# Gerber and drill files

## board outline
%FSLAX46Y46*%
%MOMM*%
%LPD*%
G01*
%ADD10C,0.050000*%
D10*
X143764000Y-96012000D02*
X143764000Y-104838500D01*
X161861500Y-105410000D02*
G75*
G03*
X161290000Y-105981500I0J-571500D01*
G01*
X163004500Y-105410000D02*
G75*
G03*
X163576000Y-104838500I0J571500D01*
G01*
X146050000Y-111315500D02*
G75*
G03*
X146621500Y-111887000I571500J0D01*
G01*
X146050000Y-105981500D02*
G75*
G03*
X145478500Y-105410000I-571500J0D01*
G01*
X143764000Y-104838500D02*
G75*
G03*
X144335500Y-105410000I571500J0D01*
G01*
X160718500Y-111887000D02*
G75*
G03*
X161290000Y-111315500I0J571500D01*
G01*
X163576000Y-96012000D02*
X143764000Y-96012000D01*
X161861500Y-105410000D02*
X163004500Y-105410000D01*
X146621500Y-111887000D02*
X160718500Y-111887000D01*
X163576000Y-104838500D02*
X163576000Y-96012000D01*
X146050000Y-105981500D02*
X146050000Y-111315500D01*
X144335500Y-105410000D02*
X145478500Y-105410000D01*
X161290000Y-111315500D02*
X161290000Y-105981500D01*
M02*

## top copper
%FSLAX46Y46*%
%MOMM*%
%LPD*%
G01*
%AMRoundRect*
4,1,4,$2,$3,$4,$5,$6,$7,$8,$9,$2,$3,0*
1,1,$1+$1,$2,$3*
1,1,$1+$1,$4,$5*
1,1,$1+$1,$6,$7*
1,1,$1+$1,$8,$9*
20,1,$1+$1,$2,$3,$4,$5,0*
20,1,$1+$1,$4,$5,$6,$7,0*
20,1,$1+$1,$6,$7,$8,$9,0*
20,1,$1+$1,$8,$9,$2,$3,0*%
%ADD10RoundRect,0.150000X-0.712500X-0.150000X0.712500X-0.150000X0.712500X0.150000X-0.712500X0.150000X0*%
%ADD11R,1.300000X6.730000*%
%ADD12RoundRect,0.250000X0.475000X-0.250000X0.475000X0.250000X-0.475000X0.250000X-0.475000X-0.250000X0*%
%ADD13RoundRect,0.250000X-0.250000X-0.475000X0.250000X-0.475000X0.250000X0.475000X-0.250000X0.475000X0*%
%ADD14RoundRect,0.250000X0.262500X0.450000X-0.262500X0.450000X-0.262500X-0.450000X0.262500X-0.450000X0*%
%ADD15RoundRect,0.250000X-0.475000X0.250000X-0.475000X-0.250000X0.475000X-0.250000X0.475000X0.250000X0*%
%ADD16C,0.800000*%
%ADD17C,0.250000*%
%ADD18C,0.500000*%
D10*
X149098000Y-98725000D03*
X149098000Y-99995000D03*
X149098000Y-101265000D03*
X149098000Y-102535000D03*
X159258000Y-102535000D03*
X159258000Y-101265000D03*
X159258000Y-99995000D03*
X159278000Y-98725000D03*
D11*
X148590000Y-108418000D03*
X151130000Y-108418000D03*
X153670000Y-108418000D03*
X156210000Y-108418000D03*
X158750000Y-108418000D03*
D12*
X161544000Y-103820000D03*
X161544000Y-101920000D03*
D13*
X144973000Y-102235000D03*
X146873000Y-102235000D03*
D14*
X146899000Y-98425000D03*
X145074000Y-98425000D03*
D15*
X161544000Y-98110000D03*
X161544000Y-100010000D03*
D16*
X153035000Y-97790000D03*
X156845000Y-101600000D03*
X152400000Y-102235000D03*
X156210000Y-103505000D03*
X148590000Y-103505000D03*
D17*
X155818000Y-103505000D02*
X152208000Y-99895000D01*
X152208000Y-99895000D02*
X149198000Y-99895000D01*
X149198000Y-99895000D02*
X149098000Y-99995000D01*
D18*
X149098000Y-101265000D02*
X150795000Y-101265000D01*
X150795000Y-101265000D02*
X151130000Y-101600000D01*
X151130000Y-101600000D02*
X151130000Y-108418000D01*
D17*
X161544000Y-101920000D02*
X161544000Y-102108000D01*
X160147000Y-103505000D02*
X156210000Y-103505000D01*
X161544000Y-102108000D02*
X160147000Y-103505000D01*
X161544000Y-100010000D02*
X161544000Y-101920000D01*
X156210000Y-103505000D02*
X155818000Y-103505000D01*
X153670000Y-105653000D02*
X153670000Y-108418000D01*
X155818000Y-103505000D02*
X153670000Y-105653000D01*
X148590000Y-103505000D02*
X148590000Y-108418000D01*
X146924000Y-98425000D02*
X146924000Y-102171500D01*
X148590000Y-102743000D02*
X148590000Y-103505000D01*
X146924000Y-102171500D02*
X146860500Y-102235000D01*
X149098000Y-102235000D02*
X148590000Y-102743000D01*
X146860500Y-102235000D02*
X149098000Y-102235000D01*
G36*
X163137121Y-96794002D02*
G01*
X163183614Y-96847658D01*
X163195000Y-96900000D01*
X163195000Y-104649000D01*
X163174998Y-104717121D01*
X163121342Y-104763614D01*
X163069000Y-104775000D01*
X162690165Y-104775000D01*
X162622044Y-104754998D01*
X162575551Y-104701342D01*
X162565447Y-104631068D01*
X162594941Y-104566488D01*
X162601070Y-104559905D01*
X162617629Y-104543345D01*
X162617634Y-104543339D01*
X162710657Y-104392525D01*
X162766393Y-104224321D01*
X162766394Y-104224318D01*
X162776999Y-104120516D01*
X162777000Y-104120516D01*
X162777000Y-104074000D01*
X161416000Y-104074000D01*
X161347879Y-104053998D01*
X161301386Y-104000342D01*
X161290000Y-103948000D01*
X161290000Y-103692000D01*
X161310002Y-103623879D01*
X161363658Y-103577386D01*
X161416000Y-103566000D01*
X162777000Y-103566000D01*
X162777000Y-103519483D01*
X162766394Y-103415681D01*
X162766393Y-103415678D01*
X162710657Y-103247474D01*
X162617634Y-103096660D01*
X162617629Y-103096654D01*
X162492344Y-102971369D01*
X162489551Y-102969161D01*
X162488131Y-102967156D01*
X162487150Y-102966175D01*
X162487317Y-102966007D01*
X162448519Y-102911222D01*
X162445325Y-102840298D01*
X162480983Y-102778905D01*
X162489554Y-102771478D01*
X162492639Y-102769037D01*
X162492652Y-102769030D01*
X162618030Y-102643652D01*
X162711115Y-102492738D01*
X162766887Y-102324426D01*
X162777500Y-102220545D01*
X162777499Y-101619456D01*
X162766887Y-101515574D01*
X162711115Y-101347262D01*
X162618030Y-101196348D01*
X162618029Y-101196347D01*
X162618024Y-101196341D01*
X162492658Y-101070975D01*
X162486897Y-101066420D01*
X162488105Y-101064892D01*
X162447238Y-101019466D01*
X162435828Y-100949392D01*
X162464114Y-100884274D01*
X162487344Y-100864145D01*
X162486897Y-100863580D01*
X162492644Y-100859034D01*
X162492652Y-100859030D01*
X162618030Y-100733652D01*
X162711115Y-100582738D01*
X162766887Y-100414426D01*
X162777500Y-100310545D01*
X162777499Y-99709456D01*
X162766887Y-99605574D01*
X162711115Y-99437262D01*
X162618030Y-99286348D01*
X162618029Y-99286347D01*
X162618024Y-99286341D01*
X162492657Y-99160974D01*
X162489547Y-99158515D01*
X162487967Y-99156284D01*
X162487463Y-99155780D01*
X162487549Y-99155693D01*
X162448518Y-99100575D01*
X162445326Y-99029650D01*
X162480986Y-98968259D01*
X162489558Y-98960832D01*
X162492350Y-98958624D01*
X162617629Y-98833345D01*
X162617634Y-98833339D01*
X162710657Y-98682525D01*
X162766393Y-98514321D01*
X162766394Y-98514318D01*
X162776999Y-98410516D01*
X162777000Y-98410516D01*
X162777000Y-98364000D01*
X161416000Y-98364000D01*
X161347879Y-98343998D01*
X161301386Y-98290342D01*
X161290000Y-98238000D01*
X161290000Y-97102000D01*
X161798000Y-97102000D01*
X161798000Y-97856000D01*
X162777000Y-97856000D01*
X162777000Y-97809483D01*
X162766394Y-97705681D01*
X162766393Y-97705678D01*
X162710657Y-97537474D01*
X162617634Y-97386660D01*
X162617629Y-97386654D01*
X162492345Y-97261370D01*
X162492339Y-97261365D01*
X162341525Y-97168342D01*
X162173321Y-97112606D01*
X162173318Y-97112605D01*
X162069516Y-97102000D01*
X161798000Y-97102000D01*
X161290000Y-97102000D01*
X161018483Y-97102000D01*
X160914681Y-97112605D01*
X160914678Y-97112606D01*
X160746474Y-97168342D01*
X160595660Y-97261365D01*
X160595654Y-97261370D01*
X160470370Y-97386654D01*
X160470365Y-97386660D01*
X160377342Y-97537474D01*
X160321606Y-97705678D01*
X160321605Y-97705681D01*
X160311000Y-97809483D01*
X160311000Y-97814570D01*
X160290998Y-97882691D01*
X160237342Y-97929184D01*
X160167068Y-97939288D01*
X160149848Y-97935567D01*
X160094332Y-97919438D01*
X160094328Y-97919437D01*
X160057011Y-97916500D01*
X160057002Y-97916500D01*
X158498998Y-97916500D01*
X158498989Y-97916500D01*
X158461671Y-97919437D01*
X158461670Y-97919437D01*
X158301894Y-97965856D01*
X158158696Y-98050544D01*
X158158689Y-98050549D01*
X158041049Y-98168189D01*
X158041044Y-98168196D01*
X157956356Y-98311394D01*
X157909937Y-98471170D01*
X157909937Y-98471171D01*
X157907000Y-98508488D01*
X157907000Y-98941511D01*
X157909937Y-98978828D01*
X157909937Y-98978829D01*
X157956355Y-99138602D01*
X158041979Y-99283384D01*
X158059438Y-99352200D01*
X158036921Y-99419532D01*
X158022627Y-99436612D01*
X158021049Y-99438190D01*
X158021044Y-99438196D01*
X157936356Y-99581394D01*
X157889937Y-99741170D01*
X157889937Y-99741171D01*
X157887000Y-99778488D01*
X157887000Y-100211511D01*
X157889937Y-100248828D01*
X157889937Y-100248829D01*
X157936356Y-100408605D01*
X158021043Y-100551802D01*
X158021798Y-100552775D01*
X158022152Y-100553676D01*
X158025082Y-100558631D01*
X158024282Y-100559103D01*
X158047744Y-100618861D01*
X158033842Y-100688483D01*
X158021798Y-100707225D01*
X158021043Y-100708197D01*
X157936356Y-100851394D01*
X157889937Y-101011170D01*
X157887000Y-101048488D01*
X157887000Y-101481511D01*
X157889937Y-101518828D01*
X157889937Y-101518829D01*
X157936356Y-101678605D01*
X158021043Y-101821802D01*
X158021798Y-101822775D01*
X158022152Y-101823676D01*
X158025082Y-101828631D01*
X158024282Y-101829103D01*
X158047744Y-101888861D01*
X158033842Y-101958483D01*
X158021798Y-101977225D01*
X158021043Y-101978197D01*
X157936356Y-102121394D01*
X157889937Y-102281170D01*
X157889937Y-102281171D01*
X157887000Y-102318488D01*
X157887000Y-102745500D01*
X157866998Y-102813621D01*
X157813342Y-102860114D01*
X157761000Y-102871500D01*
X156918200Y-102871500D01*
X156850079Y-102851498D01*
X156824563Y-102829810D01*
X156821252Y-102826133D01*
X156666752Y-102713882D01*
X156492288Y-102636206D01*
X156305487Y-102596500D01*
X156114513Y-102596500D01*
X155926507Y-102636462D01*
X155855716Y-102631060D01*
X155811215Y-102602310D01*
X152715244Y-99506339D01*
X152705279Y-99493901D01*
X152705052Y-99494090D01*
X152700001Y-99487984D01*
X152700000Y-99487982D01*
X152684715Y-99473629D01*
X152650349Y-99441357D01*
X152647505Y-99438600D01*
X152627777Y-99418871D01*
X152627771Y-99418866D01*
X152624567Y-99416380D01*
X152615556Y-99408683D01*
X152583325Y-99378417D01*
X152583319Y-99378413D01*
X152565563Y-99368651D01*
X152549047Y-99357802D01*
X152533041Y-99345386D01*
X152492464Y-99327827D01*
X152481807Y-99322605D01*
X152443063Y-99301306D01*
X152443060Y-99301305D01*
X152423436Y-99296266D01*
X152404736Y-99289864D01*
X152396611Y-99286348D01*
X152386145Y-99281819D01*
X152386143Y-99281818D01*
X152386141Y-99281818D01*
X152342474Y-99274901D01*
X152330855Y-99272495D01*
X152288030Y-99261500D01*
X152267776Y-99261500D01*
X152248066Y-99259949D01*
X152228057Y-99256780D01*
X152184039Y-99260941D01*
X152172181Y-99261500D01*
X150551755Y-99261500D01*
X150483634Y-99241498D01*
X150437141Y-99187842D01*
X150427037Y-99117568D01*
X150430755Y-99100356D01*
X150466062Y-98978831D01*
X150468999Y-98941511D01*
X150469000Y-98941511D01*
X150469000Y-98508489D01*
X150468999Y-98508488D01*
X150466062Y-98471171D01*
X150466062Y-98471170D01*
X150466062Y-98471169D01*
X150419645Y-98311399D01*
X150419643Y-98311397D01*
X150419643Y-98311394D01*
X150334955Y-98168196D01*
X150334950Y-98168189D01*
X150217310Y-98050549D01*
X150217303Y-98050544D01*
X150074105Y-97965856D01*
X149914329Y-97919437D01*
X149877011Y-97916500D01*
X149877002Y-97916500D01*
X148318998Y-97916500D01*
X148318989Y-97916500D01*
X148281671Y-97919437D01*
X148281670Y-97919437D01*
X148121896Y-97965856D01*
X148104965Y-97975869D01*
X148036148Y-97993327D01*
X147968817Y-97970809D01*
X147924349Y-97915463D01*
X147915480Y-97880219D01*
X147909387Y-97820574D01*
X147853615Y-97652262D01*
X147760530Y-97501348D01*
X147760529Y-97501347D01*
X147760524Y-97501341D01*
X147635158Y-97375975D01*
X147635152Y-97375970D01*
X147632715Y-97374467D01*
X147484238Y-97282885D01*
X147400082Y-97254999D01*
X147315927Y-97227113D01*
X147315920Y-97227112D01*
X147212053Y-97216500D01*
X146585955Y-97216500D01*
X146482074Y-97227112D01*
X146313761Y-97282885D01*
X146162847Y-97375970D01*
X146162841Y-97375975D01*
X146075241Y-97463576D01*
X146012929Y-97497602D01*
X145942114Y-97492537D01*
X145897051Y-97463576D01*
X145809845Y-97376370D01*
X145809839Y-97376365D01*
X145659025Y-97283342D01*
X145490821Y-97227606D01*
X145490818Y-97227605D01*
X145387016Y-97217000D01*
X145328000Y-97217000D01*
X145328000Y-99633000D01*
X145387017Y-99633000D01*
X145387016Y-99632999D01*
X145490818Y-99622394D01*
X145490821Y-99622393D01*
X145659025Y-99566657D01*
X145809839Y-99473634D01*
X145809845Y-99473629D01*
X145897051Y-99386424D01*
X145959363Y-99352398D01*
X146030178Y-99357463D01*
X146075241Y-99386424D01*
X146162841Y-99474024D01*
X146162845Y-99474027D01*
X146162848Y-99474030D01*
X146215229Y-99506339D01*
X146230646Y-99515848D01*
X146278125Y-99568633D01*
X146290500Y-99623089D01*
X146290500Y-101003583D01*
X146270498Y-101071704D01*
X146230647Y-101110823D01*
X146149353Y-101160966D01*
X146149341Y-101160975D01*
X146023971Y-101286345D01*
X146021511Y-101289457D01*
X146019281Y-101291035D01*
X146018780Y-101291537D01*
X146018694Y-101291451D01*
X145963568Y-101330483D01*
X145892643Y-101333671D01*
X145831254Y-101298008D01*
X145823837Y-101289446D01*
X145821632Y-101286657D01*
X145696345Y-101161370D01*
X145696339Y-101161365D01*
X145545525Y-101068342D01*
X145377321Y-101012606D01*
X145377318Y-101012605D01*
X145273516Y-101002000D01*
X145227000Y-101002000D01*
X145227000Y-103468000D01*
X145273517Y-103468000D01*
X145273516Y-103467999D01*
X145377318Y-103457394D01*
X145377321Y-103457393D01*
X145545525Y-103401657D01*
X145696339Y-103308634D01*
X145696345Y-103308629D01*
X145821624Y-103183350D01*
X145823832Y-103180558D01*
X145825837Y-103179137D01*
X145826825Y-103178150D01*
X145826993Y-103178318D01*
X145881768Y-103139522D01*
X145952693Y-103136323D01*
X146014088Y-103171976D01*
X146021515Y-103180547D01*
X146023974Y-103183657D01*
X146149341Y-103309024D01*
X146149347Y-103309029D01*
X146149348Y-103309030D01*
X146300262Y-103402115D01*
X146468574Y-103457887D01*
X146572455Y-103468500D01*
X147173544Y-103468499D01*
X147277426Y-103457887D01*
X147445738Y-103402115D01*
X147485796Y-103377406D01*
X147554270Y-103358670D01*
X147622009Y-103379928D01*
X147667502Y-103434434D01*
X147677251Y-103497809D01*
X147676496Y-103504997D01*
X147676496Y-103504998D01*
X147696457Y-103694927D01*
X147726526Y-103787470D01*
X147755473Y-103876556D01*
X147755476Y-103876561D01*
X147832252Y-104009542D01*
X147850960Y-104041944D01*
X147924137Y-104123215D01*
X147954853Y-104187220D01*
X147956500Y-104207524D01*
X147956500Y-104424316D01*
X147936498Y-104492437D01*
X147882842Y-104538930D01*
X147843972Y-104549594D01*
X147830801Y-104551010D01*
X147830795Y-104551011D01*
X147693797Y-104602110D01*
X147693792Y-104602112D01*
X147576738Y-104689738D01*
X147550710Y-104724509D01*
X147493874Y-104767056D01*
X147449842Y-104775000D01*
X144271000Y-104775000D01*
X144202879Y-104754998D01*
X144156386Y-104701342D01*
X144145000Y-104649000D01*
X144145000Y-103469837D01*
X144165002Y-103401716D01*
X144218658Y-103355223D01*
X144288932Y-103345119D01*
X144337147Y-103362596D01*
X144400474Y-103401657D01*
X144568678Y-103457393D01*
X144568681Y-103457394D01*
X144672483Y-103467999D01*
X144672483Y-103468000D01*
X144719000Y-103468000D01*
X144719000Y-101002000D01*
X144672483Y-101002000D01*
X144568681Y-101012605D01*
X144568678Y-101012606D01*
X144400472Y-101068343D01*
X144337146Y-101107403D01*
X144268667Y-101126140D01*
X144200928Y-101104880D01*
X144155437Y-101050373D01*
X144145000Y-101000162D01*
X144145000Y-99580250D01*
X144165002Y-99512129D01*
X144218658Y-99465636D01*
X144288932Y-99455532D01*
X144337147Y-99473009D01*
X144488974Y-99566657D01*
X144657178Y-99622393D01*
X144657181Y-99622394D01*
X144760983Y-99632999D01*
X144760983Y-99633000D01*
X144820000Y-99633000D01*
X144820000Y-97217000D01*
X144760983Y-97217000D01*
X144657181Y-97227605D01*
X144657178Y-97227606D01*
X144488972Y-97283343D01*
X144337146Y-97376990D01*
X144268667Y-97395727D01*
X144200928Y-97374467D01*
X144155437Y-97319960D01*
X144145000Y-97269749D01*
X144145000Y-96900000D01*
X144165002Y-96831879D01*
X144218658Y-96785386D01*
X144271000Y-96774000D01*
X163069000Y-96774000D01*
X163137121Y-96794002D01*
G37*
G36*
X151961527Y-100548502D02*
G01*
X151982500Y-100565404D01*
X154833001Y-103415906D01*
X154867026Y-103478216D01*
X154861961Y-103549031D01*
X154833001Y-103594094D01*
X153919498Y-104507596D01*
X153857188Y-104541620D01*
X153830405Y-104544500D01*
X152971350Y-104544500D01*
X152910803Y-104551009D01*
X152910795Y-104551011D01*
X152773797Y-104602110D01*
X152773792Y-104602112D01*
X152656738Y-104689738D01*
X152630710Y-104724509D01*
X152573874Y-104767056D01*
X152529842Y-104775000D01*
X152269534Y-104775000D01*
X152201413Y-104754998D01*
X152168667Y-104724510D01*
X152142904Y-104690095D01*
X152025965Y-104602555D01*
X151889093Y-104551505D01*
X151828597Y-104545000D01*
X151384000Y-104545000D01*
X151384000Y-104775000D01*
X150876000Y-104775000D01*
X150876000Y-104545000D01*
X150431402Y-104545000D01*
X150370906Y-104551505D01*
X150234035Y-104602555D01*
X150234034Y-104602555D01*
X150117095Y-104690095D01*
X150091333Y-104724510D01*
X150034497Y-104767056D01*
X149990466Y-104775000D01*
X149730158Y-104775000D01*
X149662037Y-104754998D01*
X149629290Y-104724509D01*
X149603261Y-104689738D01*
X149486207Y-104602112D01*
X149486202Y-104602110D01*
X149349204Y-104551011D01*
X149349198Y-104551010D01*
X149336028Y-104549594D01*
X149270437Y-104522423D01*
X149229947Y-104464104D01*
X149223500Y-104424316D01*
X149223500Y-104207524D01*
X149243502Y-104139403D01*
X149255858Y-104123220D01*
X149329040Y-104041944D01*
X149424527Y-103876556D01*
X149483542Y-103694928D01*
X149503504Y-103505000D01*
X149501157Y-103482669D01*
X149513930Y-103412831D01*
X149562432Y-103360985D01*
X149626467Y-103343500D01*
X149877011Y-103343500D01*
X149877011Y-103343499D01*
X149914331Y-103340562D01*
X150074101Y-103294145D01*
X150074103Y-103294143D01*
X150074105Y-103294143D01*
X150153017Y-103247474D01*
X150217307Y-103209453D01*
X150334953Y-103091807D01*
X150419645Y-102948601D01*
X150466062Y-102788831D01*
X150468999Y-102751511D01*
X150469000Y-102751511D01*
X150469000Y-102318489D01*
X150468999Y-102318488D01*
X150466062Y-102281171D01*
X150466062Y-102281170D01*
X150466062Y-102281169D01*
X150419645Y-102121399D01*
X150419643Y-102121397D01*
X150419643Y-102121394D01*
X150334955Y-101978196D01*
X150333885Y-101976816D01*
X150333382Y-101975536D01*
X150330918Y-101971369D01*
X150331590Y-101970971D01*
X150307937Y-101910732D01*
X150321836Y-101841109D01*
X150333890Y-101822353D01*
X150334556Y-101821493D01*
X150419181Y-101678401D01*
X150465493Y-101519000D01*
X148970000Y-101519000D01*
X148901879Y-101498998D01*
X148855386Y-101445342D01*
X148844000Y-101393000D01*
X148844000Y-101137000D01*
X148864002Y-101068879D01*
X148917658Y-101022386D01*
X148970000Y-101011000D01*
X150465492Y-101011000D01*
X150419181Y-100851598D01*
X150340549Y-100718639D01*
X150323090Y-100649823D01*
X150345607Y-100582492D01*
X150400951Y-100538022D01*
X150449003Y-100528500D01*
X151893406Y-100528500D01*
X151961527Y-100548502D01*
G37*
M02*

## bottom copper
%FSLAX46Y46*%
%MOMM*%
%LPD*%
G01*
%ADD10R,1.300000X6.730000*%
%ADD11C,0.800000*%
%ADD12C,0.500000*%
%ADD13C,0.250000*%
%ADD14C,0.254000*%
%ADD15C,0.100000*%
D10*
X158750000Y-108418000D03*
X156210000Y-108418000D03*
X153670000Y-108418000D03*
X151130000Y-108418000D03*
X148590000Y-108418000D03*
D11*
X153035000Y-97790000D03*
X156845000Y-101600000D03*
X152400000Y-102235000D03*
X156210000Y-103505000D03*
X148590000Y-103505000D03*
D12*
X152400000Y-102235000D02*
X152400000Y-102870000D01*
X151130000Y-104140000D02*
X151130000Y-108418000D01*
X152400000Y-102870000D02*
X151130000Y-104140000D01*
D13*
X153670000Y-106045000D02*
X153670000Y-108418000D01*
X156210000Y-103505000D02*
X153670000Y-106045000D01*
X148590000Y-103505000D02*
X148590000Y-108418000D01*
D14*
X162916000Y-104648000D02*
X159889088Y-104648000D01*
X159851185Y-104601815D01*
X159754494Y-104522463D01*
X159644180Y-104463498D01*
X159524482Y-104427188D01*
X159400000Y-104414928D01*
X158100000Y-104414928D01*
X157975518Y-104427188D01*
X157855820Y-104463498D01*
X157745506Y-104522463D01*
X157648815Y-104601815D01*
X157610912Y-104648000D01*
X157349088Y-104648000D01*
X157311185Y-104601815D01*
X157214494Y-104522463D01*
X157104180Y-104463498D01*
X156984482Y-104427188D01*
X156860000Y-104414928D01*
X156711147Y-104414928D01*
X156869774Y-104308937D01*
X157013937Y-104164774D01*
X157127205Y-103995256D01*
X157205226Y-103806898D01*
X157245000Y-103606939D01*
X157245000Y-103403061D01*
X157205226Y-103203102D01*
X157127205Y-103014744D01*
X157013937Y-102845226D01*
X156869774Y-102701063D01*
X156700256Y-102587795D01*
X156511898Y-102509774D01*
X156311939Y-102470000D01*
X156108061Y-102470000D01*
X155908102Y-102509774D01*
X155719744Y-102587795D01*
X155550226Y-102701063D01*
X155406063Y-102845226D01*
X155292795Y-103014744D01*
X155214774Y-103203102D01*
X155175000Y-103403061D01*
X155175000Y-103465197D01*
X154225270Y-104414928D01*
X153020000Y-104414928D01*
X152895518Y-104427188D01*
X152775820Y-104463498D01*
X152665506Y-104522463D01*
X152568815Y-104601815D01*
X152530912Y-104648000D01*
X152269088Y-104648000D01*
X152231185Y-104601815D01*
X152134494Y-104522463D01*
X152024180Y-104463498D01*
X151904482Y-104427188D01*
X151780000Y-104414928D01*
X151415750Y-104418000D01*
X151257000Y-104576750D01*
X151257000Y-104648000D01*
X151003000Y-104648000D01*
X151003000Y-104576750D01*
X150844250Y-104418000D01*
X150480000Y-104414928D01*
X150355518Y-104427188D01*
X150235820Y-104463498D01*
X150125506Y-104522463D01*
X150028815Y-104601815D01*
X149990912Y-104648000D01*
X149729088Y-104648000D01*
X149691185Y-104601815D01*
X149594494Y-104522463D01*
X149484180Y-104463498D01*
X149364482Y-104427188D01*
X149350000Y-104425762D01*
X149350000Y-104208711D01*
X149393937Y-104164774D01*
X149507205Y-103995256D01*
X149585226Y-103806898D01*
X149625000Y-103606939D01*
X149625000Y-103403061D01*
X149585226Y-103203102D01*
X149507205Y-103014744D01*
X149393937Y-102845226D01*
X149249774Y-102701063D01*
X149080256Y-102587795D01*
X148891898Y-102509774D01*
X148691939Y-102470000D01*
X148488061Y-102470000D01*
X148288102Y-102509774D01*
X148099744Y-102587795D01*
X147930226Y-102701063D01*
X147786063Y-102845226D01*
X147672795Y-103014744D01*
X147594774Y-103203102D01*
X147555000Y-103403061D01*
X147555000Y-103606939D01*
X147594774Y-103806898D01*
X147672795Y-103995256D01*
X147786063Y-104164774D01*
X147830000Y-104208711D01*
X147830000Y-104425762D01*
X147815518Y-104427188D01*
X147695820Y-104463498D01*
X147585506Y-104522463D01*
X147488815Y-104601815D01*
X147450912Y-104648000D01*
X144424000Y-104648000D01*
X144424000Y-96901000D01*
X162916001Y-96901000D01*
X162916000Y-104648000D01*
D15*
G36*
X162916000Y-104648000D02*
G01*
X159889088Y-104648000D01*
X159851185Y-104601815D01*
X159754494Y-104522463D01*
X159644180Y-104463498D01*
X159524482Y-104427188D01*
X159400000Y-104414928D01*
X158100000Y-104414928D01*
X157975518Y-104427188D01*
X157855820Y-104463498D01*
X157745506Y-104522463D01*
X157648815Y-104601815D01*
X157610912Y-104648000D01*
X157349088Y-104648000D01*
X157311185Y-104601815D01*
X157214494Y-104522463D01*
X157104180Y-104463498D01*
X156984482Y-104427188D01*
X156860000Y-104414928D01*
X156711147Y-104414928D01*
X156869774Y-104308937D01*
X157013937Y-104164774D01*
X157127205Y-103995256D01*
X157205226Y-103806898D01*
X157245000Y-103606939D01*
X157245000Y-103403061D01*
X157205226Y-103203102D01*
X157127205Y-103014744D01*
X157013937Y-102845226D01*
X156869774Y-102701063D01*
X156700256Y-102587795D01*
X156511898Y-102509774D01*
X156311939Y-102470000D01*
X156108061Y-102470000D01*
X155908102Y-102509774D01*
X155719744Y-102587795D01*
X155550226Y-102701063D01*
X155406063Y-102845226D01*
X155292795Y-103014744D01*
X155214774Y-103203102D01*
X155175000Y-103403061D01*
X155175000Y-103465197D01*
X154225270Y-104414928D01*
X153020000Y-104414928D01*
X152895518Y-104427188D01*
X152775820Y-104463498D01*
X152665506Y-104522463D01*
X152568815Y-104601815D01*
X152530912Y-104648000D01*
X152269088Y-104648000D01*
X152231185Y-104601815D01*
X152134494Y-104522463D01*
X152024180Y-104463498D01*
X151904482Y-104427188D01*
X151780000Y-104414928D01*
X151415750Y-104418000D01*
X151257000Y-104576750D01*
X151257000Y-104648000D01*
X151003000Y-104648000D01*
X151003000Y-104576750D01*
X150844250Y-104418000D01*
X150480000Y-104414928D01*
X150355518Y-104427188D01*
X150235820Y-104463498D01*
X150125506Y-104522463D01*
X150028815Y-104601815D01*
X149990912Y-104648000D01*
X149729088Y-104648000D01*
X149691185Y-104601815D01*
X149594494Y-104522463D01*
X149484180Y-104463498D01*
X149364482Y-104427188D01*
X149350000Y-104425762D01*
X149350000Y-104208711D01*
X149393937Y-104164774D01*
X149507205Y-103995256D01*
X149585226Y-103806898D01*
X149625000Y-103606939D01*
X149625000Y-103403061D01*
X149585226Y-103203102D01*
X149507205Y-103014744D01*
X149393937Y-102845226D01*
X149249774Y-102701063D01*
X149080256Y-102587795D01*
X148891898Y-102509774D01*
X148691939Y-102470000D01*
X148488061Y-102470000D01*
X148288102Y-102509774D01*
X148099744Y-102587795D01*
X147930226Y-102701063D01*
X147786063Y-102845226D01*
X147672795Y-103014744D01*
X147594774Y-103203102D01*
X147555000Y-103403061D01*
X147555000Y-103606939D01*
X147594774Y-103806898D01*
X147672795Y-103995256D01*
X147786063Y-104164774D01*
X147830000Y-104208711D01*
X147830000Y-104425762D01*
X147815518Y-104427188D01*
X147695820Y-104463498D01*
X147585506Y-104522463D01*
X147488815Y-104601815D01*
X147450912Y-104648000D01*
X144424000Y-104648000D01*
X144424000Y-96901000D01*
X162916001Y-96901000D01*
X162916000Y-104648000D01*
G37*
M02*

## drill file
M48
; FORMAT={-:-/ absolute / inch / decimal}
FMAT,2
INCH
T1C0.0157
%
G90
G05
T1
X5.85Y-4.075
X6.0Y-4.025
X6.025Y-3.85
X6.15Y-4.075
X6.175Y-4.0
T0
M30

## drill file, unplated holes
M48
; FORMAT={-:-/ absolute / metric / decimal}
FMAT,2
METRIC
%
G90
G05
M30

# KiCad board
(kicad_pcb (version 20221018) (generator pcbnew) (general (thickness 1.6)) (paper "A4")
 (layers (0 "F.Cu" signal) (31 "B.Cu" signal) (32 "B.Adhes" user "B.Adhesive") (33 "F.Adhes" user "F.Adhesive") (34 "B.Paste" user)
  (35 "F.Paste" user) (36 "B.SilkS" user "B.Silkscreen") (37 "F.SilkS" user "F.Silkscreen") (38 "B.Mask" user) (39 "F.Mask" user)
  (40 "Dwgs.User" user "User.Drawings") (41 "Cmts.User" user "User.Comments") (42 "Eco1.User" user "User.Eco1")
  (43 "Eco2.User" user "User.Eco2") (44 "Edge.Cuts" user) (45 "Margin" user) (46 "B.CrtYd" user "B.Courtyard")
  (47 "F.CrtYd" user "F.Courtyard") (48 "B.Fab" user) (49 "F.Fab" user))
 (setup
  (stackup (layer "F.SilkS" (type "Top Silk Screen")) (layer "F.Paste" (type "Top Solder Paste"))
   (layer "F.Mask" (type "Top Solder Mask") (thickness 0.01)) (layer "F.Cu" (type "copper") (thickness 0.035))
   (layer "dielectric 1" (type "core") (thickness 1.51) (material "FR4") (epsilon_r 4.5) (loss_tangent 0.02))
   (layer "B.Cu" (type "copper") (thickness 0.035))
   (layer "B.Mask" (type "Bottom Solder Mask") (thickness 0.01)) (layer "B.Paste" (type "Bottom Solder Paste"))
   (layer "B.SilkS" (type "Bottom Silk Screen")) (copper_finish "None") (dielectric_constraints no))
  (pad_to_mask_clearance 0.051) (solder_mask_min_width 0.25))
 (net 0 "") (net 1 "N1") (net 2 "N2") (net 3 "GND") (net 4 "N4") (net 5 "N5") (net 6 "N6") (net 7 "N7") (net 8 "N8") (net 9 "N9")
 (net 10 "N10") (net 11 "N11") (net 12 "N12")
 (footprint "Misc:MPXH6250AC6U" (layer "F.Cu") (at 154.178 100.63)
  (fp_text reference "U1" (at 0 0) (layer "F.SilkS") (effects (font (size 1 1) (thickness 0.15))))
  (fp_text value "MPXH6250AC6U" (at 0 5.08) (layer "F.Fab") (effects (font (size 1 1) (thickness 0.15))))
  (pad "1" smd roundrect (at -5.08 -1.905) (size 1.725 0.6) (layers "F.Cu" "F.Paste" "F.Mask") (roundrect_rratio 0.25) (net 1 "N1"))
  (pad "2" smd roundrect (at -5.08 -0.635) (size 1.725 0.6) (layers "F.Cu" "F.Paste" "F.Mask") (roundrect_rratio 0.25) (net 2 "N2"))
  (pad "3" smd roundrect (at -5.08 0.635) (size 1.725 0.6) (layers "F.Cu" "F.Paste" "F.Mask") (roundrect_rratio 0.25) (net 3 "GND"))
  (pad "4" smd roundrect (at -5.08 1.905) (size 1.725 0.6) (layers "F.Cu" "F.Paste" "F.Mask") (roundrect_rratio 0.25) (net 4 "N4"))
  (pad "5" smd roundrect (at 5.08 1.905) (size 1.725 0.6) (layers "F.Cu" "F.Paste" "F.Mask") (roundrect_rratio 0.25) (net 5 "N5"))
  (pad "6" smd roundrect (at 5.08 0.635) (size 1.725 0.6) (layers "F.Cu" "F.Paste" "F.Mask") (roundrect_rratio 0.25) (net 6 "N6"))
  (pad "7" smd roundrect (at 5.08 -0.635) (size 1.725 0.6) (layers "F.Cu" "F.Paste" "F.Mask") (roundrect_rratio 0.25) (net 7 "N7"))
  (pad "8" smd roundrect (at 5.1 -1.905) (size 1.725 0.6) (layers "F.Cu" "F.Paste" "F.Mask") (roundrect_rratio 0.25) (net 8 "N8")))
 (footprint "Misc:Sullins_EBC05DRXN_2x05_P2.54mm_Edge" (layer "F.Cu") (at 148.59 105.918)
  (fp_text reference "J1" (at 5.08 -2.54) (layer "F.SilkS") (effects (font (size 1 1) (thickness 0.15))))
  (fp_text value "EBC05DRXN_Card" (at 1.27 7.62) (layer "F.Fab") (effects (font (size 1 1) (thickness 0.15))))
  (pad "A1" connect rect (at 0 2.5) (size 1.3 6.73) (layers "F.Cu") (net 4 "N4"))
  (pad "A2" connect rect (at 2.54 2.5) (size 1.3 6.73) (layers "F.Cu") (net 3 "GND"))
  (pad "A3" connect rect (at 5.08 2.5) (size 1.3 6.73) (layers "F.Cu") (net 2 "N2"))
  (pad "A4" connect rect (at 7.62 2.5) (size 1.3 6.73) (layers "F.Cu") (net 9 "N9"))
  (pad "A5" connect rect (at 10.16 2.5) (size 1.3 6.73) (layers "F.Cu") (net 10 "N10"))
  (pad "B1" connect rect (at 0 2.5) (size 1.3 6.73) (layers "B.Cu") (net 4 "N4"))
  (pad "B2" connect rect (at 2.54 2.5) (size 1.3 6.73) (layers "B.Cu") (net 3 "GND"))
  (pad "B3" connect rect (at 5.08 2.5) (size 1.3 6.73) (layers "B.Cu") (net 2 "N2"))
  (pad "B4" connect rect (at 7.62 2.5) (size 1.3 6.73) (layers "B.Cu") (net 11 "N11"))
  (pad "B5" connect rect (at 10.16 2.5) (size 1.3 6.73) (layers "B.Cu") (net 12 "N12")))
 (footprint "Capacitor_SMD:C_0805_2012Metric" (layer "F.Cu") (at 161.544 102.87 90)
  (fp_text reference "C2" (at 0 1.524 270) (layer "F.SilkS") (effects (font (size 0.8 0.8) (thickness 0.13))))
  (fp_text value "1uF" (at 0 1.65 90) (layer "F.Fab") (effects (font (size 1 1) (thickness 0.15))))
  (pad "1" smd roundrect (at -0.95 0 90) (size 1 1.45) (layers "F.Cu" "F.Paste" "F.Mask") (roundrect_rratio 0.25) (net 3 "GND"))
  (pad "2" smd roundrect (at 0.95 0 90) (size 1 1.45) (layers "F.Cu" "F.Paste" "F.Mask") (roundrect_rratio 0.25) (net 2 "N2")))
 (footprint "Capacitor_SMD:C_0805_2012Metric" (layer "F.Cu") (at 145.923 102.235)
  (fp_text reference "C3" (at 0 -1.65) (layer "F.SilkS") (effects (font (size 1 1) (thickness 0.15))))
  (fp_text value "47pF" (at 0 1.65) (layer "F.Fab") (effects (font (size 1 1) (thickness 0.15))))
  (pad "1" smd roundrect (at -0.95 0) (size 1 1.45) (layers "F.Cu" "F.Paste" "F.Mask") (roundrect_rratio 0.25) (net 3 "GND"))
  (pad "2" smd roundrect (at 0.95 0) (size 1 1.45) (layers "F.Cu" "F.Paste" "F.Mask") (roundrect_rratio 0.25) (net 4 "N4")))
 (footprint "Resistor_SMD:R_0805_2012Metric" (layer "F.Cu") (at 145.9865 98.425 180)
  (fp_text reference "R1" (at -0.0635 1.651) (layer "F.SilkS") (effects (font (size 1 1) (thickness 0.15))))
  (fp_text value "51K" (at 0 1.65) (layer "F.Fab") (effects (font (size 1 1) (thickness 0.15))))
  (pad "1" smd roundrect (at -0.9125 0 180) (size 1.025 1.4) (layers "F.Cu" "F.Paste" "F.Mask") (roundrect_rratio 0.243902439) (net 4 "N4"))
  (pad "2" smd roundrect (at 0.9125 0 180) (size 1.025 1.4) (layers "F.Cu" "F.Paste" "F.Mask") (roundrect_rratio 0.243902439) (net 3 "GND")))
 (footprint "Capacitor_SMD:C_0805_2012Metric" (layer "F.Cu") (at 161.544 99.06 -90)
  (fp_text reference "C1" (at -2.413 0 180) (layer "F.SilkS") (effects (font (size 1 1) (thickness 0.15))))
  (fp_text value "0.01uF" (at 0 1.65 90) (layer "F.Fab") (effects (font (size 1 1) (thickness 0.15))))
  (pad "1" smd roundrect (at -0.95 0 270) (size 1 1.45) (layers "F.Cu" "F.Paste" "F.Mask") (roundrect_rratio 0.25) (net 3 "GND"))
  (pad "2" smd roundrect (at 0.95 0 270) (size 1 1.45) (layers "F.Cu" "F.Paste" "F.Mask") (roundrect_rratio 0.25) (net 2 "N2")))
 (gr_line (start 143.764 96.012) (end 143.764 104.8385) (stroke (width 0.05) (type solid)) (layer "Edge.Cuts"))
 (gr_arc (start 161.29 105.9815) (mid 161.457388 105.577388) (end 161.8615 105.41) (stroke (width 0.05) (type solid)) (layer "Edge.Cuts"))
 (gr_arc (start 163.576 104.8385) (mid 163.408612 105.242612) (end 163.0045 105.41) (stroke (width 0.05) (type solid)) (layer "Edge.Cuts"))
 (gr_arc (start 146.6215 111.887) (mid 146.217388 111.719612) (end 146.05 111.3155) (stroke (width 0.05) (type solid)) (layer "Edge.Cuts"))
 (gr_arc (start 145.4785 105.41) (mid 145.882612 105.577388) (end 146.05 105.9815) (stroke (width 0.05) (type solid)) (layer "Edge.Cuts"))
 (gr_arc (start 144.3355 105.41) (mid 143.931388 105.242612) (end 143.764 104.8385) (stroke (width 0.05) (type solid)) (layer "Edge.Cuts"))
 (gr_arc (start 161.29 111.3155) (mid 161.122612 111.719612) (end 160.7185 111.887) (stroke (width 0.05) (type solid)) (layer "Edge.Cuts"))
 (gr_line (start 163.576 96.012) (end 143.764 96.012) (stroke (width 0.05) (type solid)) (layer "Edge.Cuts"))
 (gr_line (start 161.8615 105.41) (end 163.0045 105.41) (stroke (width 0.05) (type solid)) (layer "Edge.Cuts"))
 (gr_line (start 146.6215 111.887) (end 160.7185 111.887) (stroke (width 0.05) (type solid)) (layer "Edge.Cuts"))
 (gr_line (start 163.576 104.8385) (end 163.576 96.012) (stroke (width 0.05) (type solid)) (layer "Edge.Cuts"))
 (gr_line (start 146.05 105.9815) (end 146.05 111.3155) (stroke (width 0.05) (type solid)) (layer "Edge.Cuts"))
 (gr_line (start 144.3355 105.41) (end 145.4785 105.41) (stroke (width 0.05) (type solid)) (layer "Edge.Cuts"))
 (gr_line (start 161.29 111.3155) (end 161.29 105.9815) (stroke (width 0.05) (type solid)) (layer "Edge.Cuts"))
 (segment (start 149.098 101.265) (end 150.795 101.265) (width 0.5) (layer "F.Cu") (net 3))
 (segment (start 150.795 101.265) (end 151.13 101.6) (width 0.5) (layer "F.Cu") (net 3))
 (segment (start 151.13 101.6) (end 151.13 108.418) (width 0.5) (layer "F.Cu") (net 3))
 (via (at 153.035 97.79) (size 0.8) (drill 0.4) (layers "F.Cu" "B.Cu") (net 3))
 (via (at 156.845 101.6) (size 0.8) (drill 0.4) (layers "F.Cu" "B.Cu") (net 3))
 (via (at 152.4 102.235) (size 0.8) (drill 0.4) (layers "F.Cu" "B.Cu") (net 3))
 (segment (start 151.13 104.14) (end 151.13 108.418) (width 0.5) (layer "B.Cu") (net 3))
 (segment (start 152.4 102.87) (end 151.13 104.14) (width 0.5) (layer "B.Cu") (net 3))
 (segment (start 152.4 102.235) (end 152.4 102.87) (width 0.5) (layer "B.Cu") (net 3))
 (segment (start 156.21 103.505) (end 155.818 103.505) (width 0.25) (layer "F.Cu") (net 2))
 (segment (start 161.544 100.01) (end 161.544 101.92) (width 0.25) (layer "F.Cu") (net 2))
 (segment (start 160.147 103.505) (end 156.21 103.505) (width 0.25) (layer "F.Cu") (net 2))
 (segment (start 161.544 102.108) (end 160.147 103.505) (width 0.25) (layer "F.Cu") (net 2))
 (segment (start 161.544 101.92) (end 161.544 102.108) (width 0.25) (layer "F.Cu") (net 2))
 (segment (start 152.208 99.895) (end 149.198 99.895) (width 0.25) (layer "F.Cu") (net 2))
 (segment (start 153.67 105.653) (end 153.67 108.418) (width 0.25) (layer "F.Cu") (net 2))
 (segment (start 155.818 103.505) (end 152.208 99.895) (width 0.25) (layer "F.Cu") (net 2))
 (segment (start 149.198 99.895) (end 149.098 99.995) (width 0.25) (layer "F.Cu") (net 2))
 (segment (start 155.818 103.505) (end 153.67 105.653) (width 0.25) (layer "F.Cu") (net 2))
 (via (at 156.21 103.505) (size 0.8) (drill 0.4) (layers "F.Cu" "B.Cu") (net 2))
 (segment (start 156.21 103.505) (end 153.67 106.045) (width 0.25) (layer "B.Cu") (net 2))
 (segment (start 153.67 106.045) (end 153.67 108.418) (width 0.25) (layer "B.Cu") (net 2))
 (segment (start 148.59 103.505) (end 148.59 108.418) (width 0.25) (layer "F.Cu") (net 4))
 (segment (start 146.924 98.425) (end 146.924 102.1715) (width 0.25) (layer "F.Cu") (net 4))
 (segment (start 148.59 102.743) (end 148.59 103.505) (width 0.25) (layer "F.Cu") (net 4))
 (segment (start 146.924 102.1715) (end 146.8605 102.235) (width 0.25) (layer "F.Cu") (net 4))
 (segment (start 149.098 102.235) (end 148.59 102.743) (width 0.25) (layer "F.Cu") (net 4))
 (segment (start 146.8605 102.235) (end 149.098 102.235) (width 0.25) (layer "F.Cu") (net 4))
 (via (at 148.59 103.505) (size 0.8) (drill 0.4) (layers "F.Cu" "B.Cu") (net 4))
 (segment (start 148.59 103.505) (end 148.59 108.418) (width 0.25) (layer "B.Cu") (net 4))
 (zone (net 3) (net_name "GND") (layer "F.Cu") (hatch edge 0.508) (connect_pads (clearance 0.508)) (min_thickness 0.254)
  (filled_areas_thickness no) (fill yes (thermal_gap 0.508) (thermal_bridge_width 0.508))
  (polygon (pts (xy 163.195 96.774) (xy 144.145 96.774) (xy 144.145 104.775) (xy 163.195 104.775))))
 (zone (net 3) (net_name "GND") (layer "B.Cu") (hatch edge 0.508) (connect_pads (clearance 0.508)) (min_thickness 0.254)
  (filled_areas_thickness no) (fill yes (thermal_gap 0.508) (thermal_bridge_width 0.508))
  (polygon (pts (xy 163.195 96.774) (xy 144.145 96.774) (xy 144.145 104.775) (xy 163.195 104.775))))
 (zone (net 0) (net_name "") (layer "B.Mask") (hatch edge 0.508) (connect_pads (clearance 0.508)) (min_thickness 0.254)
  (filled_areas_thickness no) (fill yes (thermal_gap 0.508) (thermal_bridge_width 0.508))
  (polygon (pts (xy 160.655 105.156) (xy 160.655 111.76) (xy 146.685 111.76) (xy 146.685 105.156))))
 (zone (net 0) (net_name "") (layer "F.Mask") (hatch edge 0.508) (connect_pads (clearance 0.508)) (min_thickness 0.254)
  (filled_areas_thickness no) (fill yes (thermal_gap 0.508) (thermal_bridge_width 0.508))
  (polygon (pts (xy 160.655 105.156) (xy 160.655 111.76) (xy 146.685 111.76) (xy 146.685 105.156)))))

